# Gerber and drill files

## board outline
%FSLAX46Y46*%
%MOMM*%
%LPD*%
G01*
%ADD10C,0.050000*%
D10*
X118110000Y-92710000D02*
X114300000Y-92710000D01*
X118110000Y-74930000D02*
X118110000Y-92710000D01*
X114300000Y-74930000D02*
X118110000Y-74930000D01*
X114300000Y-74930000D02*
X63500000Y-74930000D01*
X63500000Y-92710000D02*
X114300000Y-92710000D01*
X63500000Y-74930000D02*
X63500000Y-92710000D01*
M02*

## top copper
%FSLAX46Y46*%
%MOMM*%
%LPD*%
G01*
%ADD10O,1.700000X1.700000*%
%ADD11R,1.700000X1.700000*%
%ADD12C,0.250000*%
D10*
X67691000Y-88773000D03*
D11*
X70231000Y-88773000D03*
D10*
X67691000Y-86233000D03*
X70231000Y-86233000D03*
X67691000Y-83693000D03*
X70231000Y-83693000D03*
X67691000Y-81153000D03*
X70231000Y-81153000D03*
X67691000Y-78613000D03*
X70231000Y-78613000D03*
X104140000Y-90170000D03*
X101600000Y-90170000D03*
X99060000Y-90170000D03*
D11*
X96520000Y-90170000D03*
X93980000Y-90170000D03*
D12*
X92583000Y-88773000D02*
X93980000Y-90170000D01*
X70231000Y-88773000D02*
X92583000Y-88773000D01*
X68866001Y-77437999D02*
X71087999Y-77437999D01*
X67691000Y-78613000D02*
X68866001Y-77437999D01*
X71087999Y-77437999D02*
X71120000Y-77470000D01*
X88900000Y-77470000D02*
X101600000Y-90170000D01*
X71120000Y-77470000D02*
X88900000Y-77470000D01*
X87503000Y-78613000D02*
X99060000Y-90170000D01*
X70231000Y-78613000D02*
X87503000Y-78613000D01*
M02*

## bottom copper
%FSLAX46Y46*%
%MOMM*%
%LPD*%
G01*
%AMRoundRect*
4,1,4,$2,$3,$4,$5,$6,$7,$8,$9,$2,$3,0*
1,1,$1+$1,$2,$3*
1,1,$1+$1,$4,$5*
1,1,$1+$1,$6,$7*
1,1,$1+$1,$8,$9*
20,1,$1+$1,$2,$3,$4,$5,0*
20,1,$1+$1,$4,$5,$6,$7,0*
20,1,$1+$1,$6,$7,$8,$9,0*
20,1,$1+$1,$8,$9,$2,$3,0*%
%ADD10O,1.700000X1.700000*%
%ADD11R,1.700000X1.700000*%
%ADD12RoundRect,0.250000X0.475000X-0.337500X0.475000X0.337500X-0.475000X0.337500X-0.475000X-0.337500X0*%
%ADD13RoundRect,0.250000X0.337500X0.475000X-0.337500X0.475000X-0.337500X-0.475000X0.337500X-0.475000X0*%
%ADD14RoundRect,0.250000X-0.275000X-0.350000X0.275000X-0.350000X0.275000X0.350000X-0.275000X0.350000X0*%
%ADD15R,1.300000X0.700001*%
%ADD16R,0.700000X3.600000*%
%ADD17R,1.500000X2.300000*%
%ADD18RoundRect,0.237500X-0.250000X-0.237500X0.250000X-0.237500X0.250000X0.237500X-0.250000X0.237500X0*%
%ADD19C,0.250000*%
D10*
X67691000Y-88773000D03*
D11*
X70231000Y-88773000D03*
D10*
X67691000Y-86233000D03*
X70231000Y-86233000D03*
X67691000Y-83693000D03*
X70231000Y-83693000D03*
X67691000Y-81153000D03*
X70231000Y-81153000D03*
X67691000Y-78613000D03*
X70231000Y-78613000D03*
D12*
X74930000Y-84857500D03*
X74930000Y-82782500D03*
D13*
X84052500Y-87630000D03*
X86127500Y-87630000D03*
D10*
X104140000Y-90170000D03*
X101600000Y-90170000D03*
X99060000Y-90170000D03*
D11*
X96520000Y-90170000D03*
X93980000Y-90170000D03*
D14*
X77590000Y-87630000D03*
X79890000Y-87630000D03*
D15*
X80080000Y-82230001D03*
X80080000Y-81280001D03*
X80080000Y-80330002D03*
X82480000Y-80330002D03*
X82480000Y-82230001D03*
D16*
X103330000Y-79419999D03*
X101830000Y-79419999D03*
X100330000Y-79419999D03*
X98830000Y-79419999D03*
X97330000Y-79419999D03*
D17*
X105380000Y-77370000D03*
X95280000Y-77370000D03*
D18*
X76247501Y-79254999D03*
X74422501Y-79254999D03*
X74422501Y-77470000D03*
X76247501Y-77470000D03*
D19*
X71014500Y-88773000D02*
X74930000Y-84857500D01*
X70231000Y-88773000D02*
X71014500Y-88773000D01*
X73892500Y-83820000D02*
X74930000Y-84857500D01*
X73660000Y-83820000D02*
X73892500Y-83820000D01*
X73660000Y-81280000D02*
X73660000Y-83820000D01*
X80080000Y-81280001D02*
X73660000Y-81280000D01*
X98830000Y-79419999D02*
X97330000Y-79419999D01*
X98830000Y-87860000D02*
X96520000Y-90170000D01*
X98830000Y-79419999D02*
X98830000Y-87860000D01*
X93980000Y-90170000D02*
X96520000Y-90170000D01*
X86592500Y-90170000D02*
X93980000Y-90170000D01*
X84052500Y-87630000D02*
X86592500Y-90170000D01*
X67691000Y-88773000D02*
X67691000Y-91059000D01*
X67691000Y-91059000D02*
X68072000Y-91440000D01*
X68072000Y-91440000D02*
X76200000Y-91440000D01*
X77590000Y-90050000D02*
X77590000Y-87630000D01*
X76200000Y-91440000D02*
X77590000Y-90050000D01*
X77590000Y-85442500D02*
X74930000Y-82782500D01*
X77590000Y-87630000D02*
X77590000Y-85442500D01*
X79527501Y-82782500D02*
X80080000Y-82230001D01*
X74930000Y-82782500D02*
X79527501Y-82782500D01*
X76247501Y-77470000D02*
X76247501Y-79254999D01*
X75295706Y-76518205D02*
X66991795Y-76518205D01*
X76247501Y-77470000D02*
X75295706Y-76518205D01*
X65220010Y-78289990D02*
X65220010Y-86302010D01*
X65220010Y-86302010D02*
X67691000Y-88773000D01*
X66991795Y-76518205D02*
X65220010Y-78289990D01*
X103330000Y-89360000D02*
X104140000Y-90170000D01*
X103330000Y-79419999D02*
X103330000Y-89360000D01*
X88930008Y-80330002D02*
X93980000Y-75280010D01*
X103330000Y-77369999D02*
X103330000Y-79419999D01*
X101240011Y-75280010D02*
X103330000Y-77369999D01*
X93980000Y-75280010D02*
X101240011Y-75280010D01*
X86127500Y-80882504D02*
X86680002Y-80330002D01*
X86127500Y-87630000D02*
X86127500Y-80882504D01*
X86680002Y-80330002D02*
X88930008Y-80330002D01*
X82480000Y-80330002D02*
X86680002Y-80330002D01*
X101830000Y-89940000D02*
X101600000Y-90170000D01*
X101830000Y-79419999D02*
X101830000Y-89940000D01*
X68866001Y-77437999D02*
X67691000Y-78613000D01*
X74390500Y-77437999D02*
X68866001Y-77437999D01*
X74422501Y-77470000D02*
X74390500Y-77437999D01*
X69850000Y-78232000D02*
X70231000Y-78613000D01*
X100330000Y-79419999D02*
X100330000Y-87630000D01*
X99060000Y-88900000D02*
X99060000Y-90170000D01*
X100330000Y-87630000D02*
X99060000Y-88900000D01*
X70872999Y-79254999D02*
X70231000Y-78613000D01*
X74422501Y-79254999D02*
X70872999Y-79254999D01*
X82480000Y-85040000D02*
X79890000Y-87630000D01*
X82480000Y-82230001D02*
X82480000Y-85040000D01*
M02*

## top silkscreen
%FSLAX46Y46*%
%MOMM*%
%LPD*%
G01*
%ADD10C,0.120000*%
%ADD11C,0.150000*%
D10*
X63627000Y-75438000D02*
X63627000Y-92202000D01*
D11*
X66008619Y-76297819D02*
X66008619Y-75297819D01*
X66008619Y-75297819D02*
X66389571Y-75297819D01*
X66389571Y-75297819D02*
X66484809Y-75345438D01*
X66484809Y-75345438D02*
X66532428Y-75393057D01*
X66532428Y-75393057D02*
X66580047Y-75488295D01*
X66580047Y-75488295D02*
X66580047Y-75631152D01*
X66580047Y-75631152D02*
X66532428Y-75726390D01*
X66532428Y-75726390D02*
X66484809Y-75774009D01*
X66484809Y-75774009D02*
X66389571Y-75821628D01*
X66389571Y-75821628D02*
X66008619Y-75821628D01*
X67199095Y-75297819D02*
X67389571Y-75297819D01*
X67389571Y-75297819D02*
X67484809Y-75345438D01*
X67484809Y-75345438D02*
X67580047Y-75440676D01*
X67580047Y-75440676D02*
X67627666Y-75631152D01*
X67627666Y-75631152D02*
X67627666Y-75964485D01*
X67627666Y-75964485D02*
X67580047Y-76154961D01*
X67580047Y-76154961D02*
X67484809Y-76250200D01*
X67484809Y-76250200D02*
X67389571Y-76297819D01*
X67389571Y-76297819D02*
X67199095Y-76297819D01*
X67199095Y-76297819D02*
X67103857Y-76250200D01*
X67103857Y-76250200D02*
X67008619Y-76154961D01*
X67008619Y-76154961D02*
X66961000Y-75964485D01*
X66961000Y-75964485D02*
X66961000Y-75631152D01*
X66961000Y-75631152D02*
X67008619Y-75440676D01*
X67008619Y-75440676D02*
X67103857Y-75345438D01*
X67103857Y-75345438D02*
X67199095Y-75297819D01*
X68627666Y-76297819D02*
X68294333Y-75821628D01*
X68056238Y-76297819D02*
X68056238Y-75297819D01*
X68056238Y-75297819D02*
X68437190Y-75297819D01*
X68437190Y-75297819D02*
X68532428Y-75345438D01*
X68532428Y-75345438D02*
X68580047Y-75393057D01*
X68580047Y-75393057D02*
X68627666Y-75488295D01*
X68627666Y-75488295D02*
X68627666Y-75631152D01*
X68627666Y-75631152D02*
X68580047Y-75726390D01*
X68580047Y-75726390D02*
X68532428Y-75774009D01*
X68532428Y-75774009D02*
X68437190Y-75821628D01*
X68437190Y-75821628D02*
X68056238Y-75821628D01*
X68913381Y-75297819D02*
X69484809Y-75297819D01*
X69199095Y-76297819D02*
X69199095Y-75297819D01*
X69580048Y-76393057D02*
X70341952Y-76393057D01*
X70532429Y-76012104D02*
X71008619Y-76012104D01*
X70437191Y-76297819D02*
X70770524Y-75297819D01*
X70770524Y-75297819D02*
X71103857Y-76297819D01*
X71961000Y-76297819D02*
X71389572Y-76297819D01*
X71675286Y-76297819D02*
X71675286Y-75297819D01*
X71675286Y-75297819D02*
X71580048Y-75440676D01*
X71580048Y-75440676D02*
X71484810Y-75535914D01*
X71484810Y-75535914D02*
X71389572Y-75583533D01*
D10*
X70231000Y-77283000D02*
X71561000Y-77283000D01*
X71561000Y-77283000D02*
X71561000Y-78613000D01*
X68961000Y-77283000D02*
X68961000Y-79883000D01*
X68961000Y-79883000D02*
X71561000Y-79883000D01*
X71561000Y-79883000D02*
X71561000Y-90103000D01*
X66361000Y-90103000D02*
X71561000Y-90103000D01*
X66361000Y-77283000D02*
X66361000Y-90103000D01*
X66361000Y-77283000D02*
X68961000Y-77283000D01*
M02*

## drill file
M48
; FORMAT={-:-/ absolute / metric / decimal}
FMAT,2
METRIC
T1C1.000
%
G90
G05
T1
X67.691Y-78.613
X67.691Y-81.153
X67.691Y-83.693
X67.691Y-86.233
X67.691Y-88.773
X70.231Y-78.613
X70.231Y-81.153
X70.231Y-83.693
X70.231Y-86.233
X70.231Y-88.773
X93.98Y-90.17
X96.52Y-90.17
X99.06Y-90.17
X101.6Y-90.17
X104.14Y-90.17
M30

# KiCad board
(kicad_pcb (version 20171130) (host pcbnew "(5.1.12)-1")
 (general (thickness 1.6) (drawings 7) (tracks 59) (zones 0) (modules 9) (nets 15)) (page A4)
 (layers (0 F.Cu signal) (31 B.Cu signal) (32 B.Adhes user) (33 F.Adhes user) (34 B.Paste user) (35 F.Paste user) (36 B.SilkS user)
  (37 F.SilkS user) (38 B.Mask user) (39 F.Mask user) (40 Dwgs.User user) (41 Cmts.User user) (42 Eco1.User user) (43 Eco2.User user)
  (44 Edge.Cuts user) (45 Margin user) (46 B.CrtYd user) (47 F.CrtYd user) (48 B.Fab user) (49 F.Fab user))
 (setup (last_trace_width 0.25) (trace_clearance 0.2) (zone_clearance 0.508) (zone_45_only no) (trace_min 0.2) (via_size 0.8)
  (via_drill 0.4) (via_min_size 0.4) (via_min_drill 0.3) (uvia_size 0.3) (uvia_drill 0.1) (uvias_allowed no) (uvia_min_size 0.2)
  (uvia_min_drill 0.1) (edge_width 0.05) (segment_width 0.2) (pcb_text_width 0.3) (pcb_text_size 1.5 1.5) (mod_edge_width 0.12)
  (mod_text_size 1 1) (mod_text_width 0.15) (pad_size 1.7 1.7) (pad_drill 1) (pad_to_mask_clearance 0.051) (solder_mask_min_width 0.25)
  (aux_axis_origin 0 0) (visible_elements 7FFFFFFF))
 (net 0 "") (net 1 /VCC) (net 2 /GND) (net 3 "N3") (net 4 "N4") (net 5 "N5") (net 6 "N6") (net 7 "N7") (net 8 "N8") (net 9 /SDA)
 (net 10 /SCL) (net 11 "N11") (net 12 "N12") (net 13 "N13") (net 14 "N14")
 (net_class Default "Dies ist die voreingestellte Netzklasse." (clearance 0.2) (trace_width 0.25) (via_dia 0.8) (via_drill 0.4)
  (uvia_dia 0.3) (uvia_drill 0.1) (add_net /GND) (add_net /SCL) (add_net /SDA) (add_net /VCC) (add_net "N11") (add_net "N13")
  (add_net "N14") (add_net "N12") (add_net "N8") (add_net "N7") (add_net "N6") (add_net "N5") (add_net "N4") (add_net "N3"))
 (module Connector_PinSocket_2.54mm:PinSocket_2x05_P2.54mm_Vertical (layer F.Cu) (at 70.231 78.613)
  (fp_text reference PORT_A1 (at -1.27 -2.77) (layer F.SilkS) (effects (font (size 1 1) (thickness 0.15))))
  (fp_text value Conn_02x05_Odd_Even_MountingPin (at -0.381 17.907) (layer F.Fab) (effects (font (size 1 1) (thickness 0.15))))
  (fp_line (start 0 -1.33) (end 1.33 -1.33) (layer F.SilkS) (width 0.12))
  (fp_line (start 1.33 -1.33) (end 1.33 0) (layer F.SilkS) (width 0.12))
  (fp_line (start -1.27 -1.33) (end -1.27 1.27) (layer F.SilkS) (width 0.12))
  (fp_line (start -1.27 1.27) (end 1.33 1.27) (layer F.SilkS) (width 0.12))
  (fp_line (start 1.33 1.27) (end 1.33 11.49) (layer F.SilkS) (width 0.12))
  (fp_line (start -3.87 11.49) (end 1.33 11.49) (layer F.SilkS) (width 0.12))
  (fp_line (start -3.87 -1.33) (end -3.87 11.49) (layer F.SilkS) (width 0.12))
  (fp_line (start -3.87 -1.33) (end -1.27 -1.33) (layer F.SilkS) (width 0.12))
  (pad 10 thru_hole oval (at -2.54 10.16) (size 1.7 1.7) (drill 1) (layers *.Cu *.Mask) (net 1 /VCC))
  (pad 9 thru_hole rect (at 0 10.16) (size 1.7 1.7) (drill 1) (layers *.Cu *.Mask) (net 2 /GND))
  (pad 8 thru_hole oval (at -2.54 7.62) (size 1.7 1.7) (drill 1) (layers *.Cu *.Mask) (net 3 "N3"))
  (pad 7 thru_hole oval (at 0 7.62) (size 1.7 1.7) (drill 1) (layers *.Cu *.Mask) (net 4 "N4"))
  (pad 6 thru_hole oval (at -2.54 5.08) (size 1.7 1.7) (drill 1) (layers *.Cu *.Mask) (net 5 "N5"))
  (pad 5 thru_hole oval (at 0 5.08) (size 1.7 1.7) (drill 1) (layers *.Cu *.Mask) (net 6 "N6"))
  (pad 4 thru_hole oval (at -2.54 2.54) (size 1.7 1.7) (drill 1) (layers *.Cu *.Mask) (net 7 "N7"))
  (pad 3 thru_hole oval (at 0 2.54) (size 1.7 1.7) (drill 1) (layers *.Cu *.Mask) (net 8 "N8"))
  (pad 2 thru_hole oval (at -2.54 0) (size 1.7 1.7) (drill 1) (layers *.Cu *.Mask) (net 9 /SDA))
  (pad 1 thru_hole oval (at 0 0) (size 1.7 1.7) (drill 1) (layers *.Cu *.Mask) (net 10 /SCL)))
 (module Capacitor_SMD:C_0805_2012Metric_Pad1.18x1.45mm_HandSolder (layer B.Cu) (at 74.93 83.82 90)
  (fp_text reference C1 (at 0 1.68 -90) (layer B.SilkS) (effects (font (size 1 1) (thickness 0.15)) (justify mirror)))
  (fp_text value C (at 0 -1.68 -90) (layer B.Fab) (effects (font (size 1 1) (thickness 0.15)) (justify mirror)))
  (pad 1 smd roundrect (at -1.0375 0 90) (size 1.175 1.45) (layers B.Cu B.Paste B.Mask) (roundrect_rratio 0.212766) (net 2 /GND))
  (pad 2 smd roundrect (at 1.0375 0 90) (size 1.175 1.45) (layers B.Cu B.Paste B.Mask) (roundrect_rratio 0.212766) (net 1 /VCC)))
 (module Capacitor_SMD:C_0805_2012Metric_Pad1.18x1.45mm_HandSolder (layer B.Cu) (at 85.09 87.63 180)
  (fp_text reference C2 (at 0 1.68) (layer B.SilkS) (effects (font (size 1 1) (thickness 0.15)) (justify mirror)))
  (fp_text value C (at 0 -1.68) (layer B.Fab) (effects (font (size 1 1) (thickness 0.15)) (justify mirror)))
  (pad 2 smd roundrect (at 1.0375 0 180) (size 1.175 1.45) (layers B.Cu B.Paste B.Mask) (roundrect_rratio 0.212766) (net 2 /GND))
  (pad 1 smd roundrect (at -1.0375 0 180) (size 1.175 1.45) (layers B.Cu B.Paste B.Mask) (roundrect_rratio 0.212766) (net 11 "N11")))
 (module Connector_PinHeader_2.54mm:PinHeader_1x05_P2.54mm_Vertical (layer B.Cu) (at 104.14 90.17 90)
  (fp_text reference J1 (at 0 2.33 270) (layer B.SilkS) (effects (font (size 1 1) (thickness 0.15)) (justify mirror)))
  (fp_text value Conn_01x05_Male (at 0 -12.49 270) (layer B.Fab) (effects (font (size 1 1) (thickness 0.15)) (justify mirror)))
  (pad 1 thru_hole oval (at 0 0 90) (size 1.7 1.7) (drill 1) (layers *.Cu *.Mask) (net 11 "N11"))
  (pad 2 thru_hole oval (at 0 -2.54 90) (size 1.7 1.7) (drill 1) (layers *.Cu *.Mask) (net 9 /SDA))
  (pad 3 thru_hole oval (at 0 -5.08 90) (size 1.7 1.7) (drill 1) (layers *.Cu *.Mask) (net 10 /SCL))
  (pad 4 thru_hole rect (at 0 -7.62 90) (size 1.7 1.7) (drill 1) (layers *.Cu *.Mask) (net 2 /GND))
  (pad 5 thru_hole rect (at 0 -10.16 90) (size 1.7 1.7) (drill 1) (layers *.Cu *.Mask) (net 2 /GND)))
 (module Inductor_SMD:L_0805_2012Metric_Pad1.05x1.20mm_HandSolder (layer B.Cu) (at 78.74 87.63)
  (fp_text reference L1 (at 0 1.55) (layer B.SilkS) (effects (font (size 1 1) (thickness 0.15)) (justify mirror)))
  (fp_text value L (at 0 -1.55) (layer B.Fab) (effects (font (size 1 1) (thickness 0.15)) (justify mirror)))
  (pad 1 smd roundrect (at -1.15 0) (size 1.05 1.2) (layers B.Cu B.Paste B.Mask) (roundrect_rratio 0.238095) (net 1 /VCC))
  (pad 2 smd roundrect (at 1.15 0) (size 1.05 1.2) (layers B.Cu B.Paste B.Mask) (roundrect_rratio 0.238095) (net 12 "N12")))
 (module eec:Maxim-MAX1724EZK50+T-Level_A (layer B.Cu) (at 81.28 81.28)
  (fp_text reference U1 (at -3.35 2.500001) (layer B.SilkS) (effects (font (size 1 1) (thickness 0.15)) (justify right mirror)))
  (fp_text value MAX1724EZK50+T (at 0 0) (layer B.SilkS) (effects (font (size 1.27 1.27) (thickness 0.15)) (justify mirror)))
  (pad 1 smd rect (at -1.2 0.950001 90) (size 0.700001 1.3) (layers B.Cu B.Paste B.Mask) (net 1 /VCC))
  (pad 2 smd rect (at -1.2 0.000001 90) (size 0.700001 1.3) (layers B.Cu B.Paste B.Mask) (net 2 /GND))
  (pad 3 smd rect (at -1.2 -0.949998 90) (size 0.700001 1.3) (layers B.Cu B.Paste B.Mask) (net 1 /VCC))
  (pad 4 smd rect (at 1.2 -0.949998 90) (size 0.700001 1.3) (layers B.Cu B.Paste B.Mask) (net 11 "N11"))
  (pad 5 smd rect (at 1.2 0.950001 90) (size 0.700001 1.3) (layers B.Cu B.Paste B.Mask) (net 12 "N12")))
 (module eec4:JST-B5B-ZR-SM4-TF (layer B.Cu) (at 100.33 77.47 180)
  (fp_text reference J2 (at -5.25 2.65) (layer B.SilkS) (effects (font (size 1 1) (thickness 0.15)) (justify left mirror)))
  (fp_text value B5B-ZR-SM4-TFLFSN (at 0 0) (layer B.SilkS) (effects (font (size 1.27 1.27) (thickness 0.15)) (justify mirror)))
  (pad 1 smd rect (at -3 -1.949999 180) (size 0.7 3.6) (layers B.Cu B.Paste B.Mask) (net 11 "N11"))
  (pad 2 smd rect (at -1.5 -1.949999 180) (size 0.7 3.6) (layers B.Cu B.Paste B.Mask) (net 9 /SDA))
  (pad 3 smd rect (at 0 -1.949999 180) (size 0.7 3.6) (layers B.Cu B.Paste B.Mask) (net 10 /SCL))
  (pad 4 smd rect (at 1.5 -1.949999 180) (size 0.7 3.6) (layers B.Cu B.Paste B.Mask) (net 2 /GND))
  (pad 5 smd rect (at 3 -1.949999 180) (size 0.7 3.6) (layers B.Cu B.Paste B.Mask) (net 2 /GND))
  (pad 6 smd rect (at -5.05 0.1 180) (size 1.5 2.3) (layers B.Cu B.Paste B.Mask) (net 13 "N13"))
  (pad 7 smd rect (at 5.05 0.1 180) (size 1.5 2.3) (layers B.Cu B.Paste B.Mask) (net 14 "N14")))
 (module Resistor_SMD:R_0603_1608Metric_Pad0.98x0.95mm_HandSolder (layer B.Cu) (at 75.335001 79.254999)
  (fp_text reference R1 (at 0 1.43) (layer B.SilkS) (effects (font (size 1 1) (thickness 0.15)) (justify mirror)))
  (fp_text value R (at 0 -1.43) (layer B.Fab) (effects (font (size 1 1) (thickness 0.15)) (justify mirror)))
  (pad 2 smd roundrect (at 0.9125 0) (size 0.975 0.95) (layers B.Cu B.Paste B.Mask) (roundrect_rratio 0.25) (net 1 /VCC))
  (pad 1 smd roundrect (at -0.9125 0) (size 0.975 0.95) (layers B.Cu B.Paste B.Mask) (roundrect_rratio 0.25) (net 10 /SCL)))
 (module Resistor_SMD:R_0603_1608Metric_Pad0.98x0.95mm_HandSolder (layer B.Cu) (at 75.335001 77.47)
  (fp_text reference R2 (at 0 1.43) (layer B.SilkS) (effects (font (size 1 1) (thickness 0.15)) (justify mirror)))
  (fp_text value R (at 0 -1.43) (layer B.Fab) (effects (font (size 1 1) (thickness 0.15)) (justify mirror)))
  (pad 1 smd roundrect (at -0.9125 0) (size 0.975 0.95) (layers B.Cu B.Paste B.Mask) (roundrect_rratio 0.25) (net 9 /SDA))
  (pad 2 smd roundrect (at 0.9125 0) (size 0.975 0.95) (layers B.Cu B.Paste B.Mask) (roundrect_rratio 0.25) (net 1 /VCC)))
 (gr_line (start 118.11 92.71) (end 114.3 92.71) (layer Edge.Cuts) (width 0.05))
 (gr_line (start 118.11 74.93) (end 118.11 92.71) (layer Edge.Cuts) (width 0.05))
 (gr_line (start 114.3 74.93) (end 118.11 74.93) (layer Edge.Cuts) (width 0.05))
 (gr_line (start 114.3 74.93) (end 63.5 74.93) (layer Edge.Cuts) (width 0.05))
 (gr_line (start 63.5 92.71) (end 114.3 92.71) (layer Edge.Cuts) (width 0.05))
 (gr_line (start 63.5 74.93) (end 63.5 92.71) (layer Edge.Cuts) (width 0.05))
 (gr_line (start 63.627 75.438) (end 63.627 92.202) (layer F.SilkS) (width 0.12))
 (segment (start 71.0145 88.773) (end 74.93 84.8575) (width 0.25) (layer B.Cu) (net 2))
 (segment (start 70.231 88.773) (end 71.0145 88.773) (width 0.25) (layer B.Cu) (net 2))
 (segment (start 73.8925 83.82) (end 74.93 84.8575) (width 0.25) (layer B.Cu) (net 2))
 (segment (start 73.66 83.82) (end 73.8925 83.82) (width 0.25) (layer B.Cu) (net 2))
 (segment (start 73.66 81.28) (end 73.66 83.82) (width 0.25) (layer B.Cu) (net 2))
 (segment (start 80.08 81.280001) (end 73.66 81.28) (width 0.25) (layer B.Cu) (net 2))
 (segment (start 98.83 79.419999) (end 97.33 79.419999) (width 0.25) (layer B.Cu) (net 2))
 (segment (start 98.83 87.86) (end 96.52 90.17) (width 0.25) (layer B.Cu) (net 2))
 (segment (start 98.83 79.419999) (end 98.83 87.86) (width 0.25) (layer B.Cu) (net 2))
 (segment (start 93.98 90.17) (end 96.52 90.17) (width 0.25) (layer B.Cu) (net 2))
 (segment (start 92.583 88.773) (end 93.98 90.17) (width 0.25) (layer F.Cu) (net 2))
 (segment (start 70.231 88.773) (end 92.583 88.773) (width 0.25) (layer F.Cu) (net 2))
 (segment (start 86.5925 90.17) (end 93.98 90.17) (width 0.25) (layer B.Cu) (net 2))
 (segment (start 84.0525 87.63) (end 86.5925 90.17) (width 0.25) (layer B.Cu) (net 2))
 (segment (start 67.691 88.773) (end 67.691 91.059) (width 0.25) (layer B.Cu) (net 1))
 (segment (start 67.691 91.059) (end 68.072 91.44) (width 0.25) (layer B.Cu) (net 1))
 (segment (start 68.072 91.44) (end 76.2 91.44) (width 0.25) (layer B.Cu) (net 1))
 (segment (start 77.59 90.05) (end 77.59 87.63) (width 0.25) (layer B.Cu) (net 1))
 (segment (start 76.2 91.44) (end 77.59 90.05) (width 0.25) (layer B.Cu) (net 1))
 (segment (start 77.59 85.4425) (end 74.93 82.7825) (width 0.25) (layer B.Cu) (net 1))
 (segment (start 77.59 87.63) (end 77.59 85.4425) (width 0.25) (layer B.Cu) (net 1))
 (segment (start 79.527501 82.7825) (end 80.08 82.230001) (width 0.25) (layer B.Cu) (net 1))
 (segment (start 74.93 82.7825) (end 79.527501 82.7825) (width 0.25) (layer B.Cu) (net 1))
 (segment (start 76.247501 77.47) (end 76.247501 79.254999) (width 0.25) (layer B.Cu) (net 1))
 (segment (start 75.295706 76.518205) (end 66.991795 76.518205) (width 0.25) (layer B.Cu) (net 1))
 (segment (start 76.247501 77.47) (end 75.295706 76.518205) (width 0.25) (layer B.Cu) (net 1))
 (segment (start 65.22001 78.28999) (end 65.22001 86.30201) (width 0.25) (layer B.Cu) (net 1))
 (segment (start 65.22001 86.30201) (end 67.691 88.773) (width 0.25) (layer B.Cu) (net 1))
 (segment (start 66.991795 76.518205) (end 65.22001 78.28999) (width 0.25) (layer B.Cu) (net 1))
 (segment (start 103.33 89.36) (end 104.14 90.17) (width 0.25) (layer B.Cu) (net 11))
 (segment (start 103.33 79.419999) (end 103.33 89.36) (width 0.25) (layer B.Cu) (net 11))
 (segment (start 88.930008 80.330002) (end 93.98 75.28001) (width 0.25) (layer B.Cu) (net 11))
 (segment (start 103.33 77.369999) (end 103.33 79.419999) (width 0.25) (layer B.Cu) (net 11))
 (segment (start 101.240011 75.28001) (end 103.33 77.369999) (width 0.25) (layer B.Cu) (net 11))
 (segment (start 93.98 75.28001) (end 101.240011 75.28001) (width 0.25) (layer B.Cu) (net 11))
 (segment (start 86.1275 80.882504) (end 86.680002 80.330002) (width 0.25) (layer B.Cu) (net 11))
 (segment (start 86.1275 87.63) (end 86.1275 80.882504) (width 0.25) (layer B.Cu) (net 11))
 (segment (start 86.680002 80.330002) (end 88.930008 80.330002) (width 0.25) (layer B.Cu) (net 11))
 (segment (start 82.48 80.330002) (end 86.680002 80.330002) (width 0.25) (layer B.Cu) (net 11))
 (segment (start 101.83 89.94) (end 101.6 90.17) (width 0.25) (layer B.Cu) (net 9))
 (segment (start 101.83 79.419999) (end 101.83 89.94) (width 0.25) (layer B.Cu) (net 9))
 (segment (start 68.866001 77.437999) (end 71.087999 77.437999) (width 0.25) (layer F.Cu) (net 9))
 (segment (start 67.691 78.613) (end 68.866001 77.437999) (width 0.25) (layer F.Cu) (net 9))
 (segment (start 71.087999 77.437999) (end 71.12 77.47) (width 0.25) (layer F.Cu) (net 9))
 (segment (start 88.9 77.47) (end 101.6 90.17) (width 0.25) (layer F.Cu) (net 9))
 (segment (start 71.12 77.47) (end 88.9 77.47) (width 0.25) (layer F.Cu) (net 9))
 (segment (start 68.866001 77.437999) (end 67.691 78.613) (width 0.25) (layer B.Cu) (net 9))
 (segment (start 74.3905 77.437999) (end 68.866001 77.437999) (width 0.25) (layer B.Cu) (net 9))
 (segment (start 74.422501 77.47) (end 74.3905 77.437999) (width 0.25) (layer B.Cu) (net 9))
 (segment (start 69.85 78.232) (end 70.231 78.613) (width 0.25) (layer B.Cu) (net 10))
 (segment (start 100.33 79.419999) (end 100.33 87.63) (width 0.25) (layer B.Cu) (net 10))
 (segment (start 99.06 88.9) (end 99.06 90.17) (width 0.25) (layer B.Cu) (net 10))
 (segment (start 100.33 87.63) (end 99.06 88.9) (width 0.25) (layer B.Cu) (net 10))
 (segment (start 87.503 78.613) (end 99.06 90.17) (width 0.25) (layer F.Cu) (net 10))
 (segment (start 70.231 78.613) (end 87.503 78.613) (width 0.25) (layer F.Cu) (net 10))
 (segment (start 70.872999 79.254999) (end 70.231 78.613) (width 0.25) (layer B.Cu) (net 10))
 (segment (start 74.422501 79.254999) (end 70.872999 79.254999) (width 0.25) (layer B.Cu) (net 10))
 (segment (start 82.48 85.04) (end 79.89 87.63) (width 0.25) (layer B.Cu) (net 12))
 (segment (start 82.48 82.230001) (end 82.48 85.04) (width 0.25) (layer B.Cu) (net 12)))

